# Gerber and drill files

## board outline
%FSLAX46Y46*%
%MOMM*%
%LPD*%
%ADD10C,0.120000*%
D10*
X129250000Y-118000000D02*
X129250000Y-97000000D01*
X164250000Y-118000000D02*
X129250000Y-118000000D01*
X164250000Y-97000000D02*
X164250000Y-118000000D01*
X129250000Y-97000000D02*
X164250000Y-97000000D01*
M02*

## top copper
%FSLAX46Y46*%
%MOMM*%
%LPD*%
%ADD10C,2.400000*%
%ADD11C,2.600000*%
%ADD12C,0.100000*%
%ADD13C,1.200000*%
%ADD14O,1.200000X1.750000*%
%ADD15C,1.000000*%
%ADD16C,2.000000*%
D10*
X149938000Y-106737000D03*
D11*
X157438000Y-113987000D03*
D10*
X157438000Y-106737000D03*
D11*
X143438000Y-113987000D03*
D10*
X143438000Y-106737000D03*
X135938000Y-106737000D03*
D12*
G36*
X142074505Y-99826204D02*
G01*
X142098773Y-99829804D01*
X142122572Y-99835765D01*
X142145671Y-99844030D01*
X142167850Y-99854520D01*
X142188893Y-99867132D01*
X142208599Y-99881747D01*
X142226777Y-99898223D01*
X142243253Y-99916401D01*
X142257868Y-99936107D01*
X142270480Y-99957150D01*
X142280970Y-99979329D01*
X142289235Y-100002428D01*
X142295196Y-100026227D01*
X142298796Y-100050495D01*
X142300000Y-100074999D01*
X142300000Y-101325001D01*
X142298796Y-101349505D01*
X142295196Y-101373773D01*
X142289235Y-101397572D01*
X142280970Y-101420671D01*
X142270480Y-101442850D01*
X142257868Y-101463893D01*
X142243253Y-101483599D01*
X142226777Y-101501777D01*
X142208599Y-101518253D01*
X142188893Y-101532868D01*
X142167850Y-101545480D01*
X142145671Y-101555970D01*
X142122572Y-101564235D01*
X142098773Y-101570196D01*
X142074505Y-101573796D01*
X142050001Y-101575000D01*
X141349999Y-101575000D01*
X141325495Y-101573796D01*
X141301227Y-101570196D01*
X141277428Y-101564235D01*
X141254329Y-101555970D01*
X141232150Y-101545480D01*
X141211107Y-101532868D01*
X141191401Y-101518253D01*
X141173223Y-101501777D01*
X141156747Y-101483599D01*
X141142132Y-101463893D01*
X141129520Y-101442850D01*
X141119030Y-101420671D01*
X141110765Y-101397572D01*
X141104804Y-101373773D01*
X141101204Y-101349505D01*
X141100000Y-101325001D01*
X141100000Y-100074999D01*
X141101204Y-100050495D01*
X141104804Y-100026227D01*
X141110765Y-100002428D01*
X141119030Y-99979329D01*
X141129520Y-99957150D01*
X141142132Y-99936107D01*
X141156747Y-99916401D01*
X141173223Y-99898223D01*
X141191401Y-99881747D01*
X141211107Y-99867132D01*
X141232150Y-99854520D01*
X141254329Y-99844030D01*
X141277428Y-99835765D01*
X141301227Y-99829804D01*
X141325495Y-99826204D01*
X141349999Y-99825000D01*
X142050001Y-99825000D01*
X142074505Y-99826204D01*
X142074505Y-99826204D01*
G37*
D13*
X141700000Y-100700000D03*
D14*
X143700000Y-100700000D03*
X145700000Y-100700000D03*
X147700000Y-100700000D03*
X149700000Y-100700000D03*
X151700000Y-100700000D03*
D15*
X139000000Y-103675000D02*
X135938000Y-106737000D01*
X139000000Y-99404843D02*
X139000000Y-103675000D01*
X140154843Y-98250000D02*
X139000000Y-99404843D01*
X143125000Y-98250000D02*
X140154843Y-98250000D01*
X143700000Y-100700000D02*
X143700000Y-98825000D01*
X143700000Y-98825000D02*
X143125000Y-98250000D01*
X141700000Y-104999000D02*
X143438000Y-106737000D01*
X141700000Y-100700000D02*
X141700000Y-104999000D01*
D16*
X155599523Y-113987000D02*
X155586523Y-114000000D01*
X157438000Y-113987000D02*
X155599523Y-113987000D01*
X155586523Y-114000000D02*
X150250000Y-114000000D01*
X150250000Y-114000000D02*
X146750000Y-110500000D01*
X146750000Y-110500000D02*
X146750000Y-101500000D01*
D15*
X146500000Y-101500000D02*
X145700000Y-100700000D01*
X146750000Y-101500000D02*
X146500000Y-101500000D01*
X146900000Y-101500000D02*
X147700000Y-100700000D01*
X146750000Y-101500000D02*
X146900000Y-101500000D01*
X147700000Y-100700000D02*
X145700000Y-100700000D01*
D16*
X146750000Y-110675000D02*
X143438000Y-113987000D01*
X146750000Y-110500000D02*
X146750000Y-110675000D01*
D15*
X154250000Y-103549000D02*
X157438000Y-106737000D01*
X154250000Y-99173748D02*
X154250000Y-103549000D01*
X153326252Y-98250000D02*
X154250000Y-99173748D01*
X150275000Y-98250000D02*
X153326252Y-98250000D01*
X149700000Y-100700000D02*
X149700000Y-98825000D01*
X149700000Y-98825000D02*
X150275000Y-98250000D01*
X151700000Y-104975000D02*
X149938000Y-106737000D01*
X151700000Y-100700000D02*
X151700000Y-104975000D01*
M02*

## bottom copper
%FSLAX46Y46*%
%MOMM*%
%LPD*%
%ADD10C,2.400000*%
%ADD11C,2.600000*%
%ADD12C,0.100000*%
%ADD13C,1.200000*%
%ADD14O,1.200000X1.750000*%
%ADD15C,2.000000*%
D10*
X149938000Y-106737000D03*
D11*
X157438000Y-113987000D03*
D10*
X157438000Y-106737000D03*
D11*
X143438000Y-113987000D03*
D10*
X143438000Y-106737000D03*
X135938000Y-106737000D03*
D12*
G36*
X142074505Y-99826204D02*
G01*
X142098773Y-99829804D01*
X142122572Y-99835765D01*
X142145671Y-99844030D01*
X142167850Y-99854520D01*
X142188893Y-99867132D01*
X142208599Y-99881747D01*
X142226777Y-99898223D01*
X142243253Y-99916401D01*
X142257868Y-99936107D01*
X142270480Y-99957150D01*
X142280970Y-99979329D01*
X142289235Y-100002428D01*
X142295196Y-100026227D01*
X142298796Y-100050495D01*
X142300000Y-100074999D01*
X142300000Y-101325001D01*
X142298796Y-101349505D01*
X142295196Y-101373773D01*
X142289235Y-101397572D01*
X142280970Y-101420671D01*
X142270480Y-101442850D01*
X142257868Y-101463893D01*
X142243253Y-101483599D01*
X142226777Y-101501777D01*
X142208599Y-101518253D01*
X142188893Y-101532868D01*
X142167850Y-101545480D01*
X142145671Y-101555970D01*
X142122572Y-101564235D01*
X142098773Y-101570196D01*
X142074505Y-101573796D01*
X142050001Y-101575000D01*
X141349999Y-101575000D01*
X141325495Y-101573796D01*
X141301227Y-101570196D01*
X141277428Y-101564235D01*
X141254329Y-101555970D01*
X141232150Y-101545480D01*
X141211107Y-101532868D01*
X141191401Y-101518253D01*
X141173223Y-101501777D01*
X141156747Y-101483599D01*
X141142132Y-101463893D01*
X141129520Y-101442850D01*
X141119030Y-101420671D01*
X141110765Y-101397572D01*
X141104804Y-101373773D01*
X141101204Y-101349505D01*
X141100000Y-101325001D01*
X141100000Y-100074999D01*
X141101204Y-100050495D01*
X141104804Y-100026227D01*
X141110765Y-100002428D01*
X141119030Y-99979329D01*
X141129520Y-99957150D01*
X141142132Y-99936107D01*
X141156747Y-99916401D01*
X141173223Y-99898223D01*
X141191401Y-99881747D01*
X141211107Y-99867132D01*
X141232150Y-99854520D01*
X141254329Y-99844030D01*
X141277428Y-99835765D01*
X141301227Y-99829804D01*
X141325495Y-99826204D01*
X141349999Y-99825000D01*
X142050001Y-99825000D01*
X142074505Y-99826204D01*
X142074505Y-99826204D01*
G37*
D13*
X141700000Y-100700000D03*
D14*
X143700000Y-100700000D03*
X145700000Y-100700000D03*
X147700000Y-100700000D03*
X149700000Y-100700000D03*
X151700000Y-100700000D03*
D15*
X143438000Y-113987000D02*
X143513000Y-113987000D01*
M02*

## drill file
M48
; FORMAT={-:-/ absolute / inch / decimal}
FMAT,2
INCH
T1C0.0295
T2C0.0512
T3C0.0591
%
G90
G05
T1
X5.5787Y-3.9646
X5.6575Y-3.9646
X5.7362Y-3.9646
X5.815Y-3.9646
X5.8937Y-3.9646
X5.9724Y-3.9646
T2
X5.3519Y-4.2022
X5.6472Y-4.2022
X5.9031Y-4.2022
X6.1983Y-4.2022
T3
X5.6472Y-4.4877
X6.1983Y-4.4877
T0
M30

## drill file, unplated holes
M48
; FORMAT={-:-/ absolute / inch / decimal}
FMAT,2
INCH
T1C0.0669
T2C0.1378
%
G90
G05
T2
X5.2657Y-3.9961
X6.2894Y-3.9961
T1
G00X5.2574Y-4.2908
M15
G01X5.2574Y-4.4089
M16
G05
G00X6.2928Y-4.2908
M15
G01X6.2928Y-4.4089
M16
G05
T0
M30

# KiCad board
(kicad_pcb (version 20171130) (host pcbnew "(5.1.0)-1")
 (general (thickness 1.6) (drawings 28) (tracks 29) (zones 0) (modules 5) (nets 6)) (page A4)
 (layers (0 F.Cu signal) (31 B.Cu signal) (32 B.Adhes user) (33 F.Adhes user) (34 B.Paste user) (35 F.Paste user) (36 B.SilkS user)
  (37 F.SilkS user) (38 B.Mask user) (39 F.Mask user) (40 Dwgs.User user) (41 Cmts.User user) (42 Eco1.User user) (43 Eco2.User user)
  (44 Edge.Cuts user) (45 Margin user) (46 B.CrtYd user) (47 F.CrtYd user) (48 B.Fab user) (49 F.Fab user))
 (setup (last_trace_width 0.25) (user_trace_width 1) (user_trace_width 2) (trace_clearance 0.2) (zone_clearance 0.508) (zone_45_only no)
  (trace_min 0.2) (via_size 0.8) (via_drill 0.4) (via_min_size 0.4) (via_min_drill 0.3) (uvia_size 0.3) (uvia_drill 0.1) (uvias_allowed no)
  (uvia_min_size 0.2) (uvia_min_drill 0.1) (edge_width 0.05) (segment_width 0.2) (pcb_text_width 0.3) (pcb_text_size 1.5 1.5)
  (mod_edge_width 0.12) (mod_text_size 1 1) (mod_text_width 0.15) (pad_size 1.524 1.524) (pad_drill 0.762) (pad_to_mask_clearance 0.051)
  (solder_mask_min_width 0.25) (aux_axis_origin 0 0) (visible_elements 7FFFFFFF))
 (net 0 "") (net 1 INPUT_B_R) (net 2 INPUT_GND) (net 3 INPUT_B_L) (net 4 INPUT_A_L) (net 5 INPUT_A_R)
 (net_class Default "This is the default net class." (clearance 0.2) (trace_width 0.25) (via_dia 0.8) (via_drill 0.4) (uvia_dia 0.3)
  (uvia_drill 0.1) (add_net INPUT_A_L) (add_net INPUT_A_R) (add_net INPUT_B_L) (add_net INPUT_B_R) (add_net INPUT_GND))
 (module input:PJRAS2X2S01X (layer F.Cu) (at 135.938 106.737)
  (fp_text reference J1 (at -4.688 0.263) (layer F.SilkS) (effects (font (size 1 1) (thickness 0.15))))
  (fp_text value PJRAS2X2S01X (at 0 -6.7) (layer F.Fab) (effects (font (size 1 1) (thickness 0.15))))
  (pad "" np_thru_hole oval (at 23.9 3.75) (size 1.7 4.7) (drill oval 1.7 4.7) (layers *.Cu *.Mask))
  (pad "" np_thru_hole oval (at -2.4 3.75) (size 1.7 4.7) (drill oval 1.7 4.7) (layers *.Cu *.Mask))
  (pad 4 thru_hole circle (at 14 0) (size 2.4 2.4) (drill 1.3) (layers *.Cu *.Mask) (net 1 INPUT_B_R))
  (pad 5 thru_hole circle (at 21.5 7.25) (size 2.6 2.6) (drill 1.5) (layers *.Cu *.Mask) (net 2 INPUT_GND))
  (pad 6 thru_hole circle (at 21.5 0) (size 2.4 2.4) (drill 1.3) (layers *.Cu *.Mask) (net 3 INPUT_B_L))
  (pad 2 thru_hole circle (at 7.5 7.25) (size 2.6 2.6) (drill 1.5) (layers *.Cu *.Mask) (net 2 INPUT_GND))
  (pad 3 thru_hole circle (at 7.5 0) (size 2.4 2.4) (drill 1.3) (layers *.Cu *.Mask) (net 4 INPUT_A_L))
  (pad 1 thru_hole circle (at 0 0) (size 2.4 2.4) (drill 1.3) (layers *.Cu *.Mask) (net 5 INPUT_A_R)))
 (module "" (layer F.Cu) (at 140.5 94.25)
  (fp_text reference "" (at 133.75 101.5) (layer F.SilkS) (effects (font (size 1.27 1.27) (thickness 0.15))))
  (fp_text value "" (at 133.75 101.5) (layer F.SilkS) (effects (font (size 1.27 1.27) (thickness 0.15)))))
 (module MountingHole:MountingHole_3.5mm (layer F.Cu) (at 133.75 101.5)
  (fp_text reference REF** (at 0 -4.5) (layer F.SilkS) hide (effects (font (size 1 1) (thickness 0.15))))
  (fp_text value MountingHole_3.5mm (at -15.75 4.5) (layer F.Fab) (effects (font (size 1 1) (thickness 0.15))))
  (pad 1 np_thru_hole circle (at 0 0) (size 3.5 3.5) (drill 3.5) (layers *.Cu *.Mask)))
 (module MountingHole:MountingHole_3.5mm (layer F.Cu) (at 159.75 101.5)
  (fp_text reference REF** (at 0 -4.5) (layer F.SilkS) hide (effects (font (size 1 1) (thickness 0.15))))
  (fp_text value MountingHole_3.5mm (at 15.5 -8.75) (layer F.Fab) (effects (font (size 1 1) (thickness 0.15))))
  (pad 1 np_thru_hole circle (at 0 0) (size 3.5 3.5) (drill 3.5) (layers *.Cu *.Mask)))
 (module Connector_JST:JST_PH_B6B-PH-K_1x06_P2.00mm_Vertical (layer F.Cu) (at 141.7 100.7)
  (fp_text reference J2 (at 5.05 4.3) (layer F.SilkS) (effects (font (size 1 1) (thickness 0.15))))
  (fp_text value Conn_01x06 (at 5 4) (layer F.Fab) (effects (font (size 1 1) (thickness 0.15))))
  (pad 1 thru_hole roundrect (at 0 0) (size 1.2 1.75) (drill 0.75) (layers *.Cu *.Mask) (roundrect_rratio 0.208333) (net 4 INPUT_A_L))
  (pad 2 thru_hole oval (at 2 0) (size 1.2 1.75) (drill 0.75) (layers *.Cu *.Mask) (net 5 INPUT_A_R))
  (pad 3 thru_hole oval (at 4 0) (size 1.2 1.75) (drill 0.75) (layers *.Cu *.Mask) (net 2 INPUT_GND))
  (pad 4 thru_hole oval (at 6 0) (size 1.2 1.75) (drill 0.75) (layers *.Cu *.Mask) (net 2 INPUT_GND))
  (pad 5 thru_hole oval (at 8 0) (size 1.2 1.75) (drill 0.75) (layers *.Cu *.Mask) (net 3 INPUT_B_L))
  (pad 6 thru_hole oval (at 10 0) (size 1.2 1.75) (drill 0.75) (layers *.Cu *.Mask) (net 1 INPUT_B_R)))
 (gr_line (start 129.25 118) (end 129.25 97) (layer Edge.Cuts) (width 0.12))
 (gr_line (start 164.25 118) (end 129.25 118) (layer Edge.Cuts) (width 0.12))
 (gr_line (start 164.25 97) (end 164.25 118) (layer Edge.Cuts) (width 0.12))
 (gr_line (start 129.25 97) (end 164.25 97) (layer Edge.Cuts) (width 0.12))
 (segment (start 139 103.675) (end 135.938 106.737) (width 1) (layer F.Cu) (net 5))
 (segment (start 139 99.404843) (end 139 103.675) (width 1) (layer F.Cu) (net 5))
 (segment (start 140.154843 98.25) (end 139 99.404843) (width 1) (layer F.Cu) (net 5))
 (segment (start 143.125 98.25) (end 140.154843 98.25) (width 1) (layer F.Cu) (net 5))
 (segment (start 143.7 100.7) (end 143.7 98.825) (width 1) (layer F.Cu) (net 5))
 (segment (start 143.7 98.825) (end 143.125 98.25) (width 1) (layer F.Cu) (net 5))
 (segment (start 141.7 104.999) (end 143.438 106.737) (width 1) (layer F.Cu) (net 4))
 (segment (start 141.7 100.7) (end 141.7 104.999) (width 1) (layer F.Cu) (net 4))
 (segment (start 155.599523 113.987) (end 155.586523 114) (width 2) (layer F.Cu) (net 2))
 (segment (start 157.438 113.987) (end 155.599523 113.987) (width 2) (layer F.Cu) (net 2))
 (segment (start 155.586523 114) (end 150.25 114) (width 2) (layer F.Cu) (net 2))
 (segment (start 150.25 114) (end 146.75 110.5) (width 2) (layer F.Cu) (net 2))
 (segment (start 146.75 110.5) (end 146.75 101.5) (width 2) (layer F.Cu) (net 2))
 (segment (start 146.5 101.5) (end 145.7 100.7) (width 1) (layer F.Cu) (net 2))
 (segment (start 146.75 101.5) (end 146.5 101.5) (width 1) (layer F.Cu) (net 2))
 (segment (start 146.9 101.5) (end 147.7 100.7) (width 1) (layer F.Cu) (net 2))
 (segment (start 146.75 101.5) (end 146.9 101.5) (width 1) (layer F.Cu) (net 2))
 (segment (start 143.438 113.987) (end 143.513 113.987) (width 2) (layer B.Cu) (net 2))
 (segment (start 147.7 100.7) (end 145.7 100.7) (width 1) (layer F.Cu) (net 2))
 (segment (start 146.75 110.675) (end 143.438 113.987) (width 2) (layer F.Cu) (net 2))
 (segment (start 146.75 110.5) (end 146.75 110.675) (width 2) (layer F.Cu) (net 2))
 (segment (start 154.25 103.549) (end 157.438 106.737) (width 1) (layer F.Cu) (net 3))
 (segment (start 154.25 99.173748) (end 154.25 103.549) (width 1) (layer F.Cu) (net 3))
 (segment (start 153.326252 98.25) (end 154.25 99.173748) (width 1) (layer F.Cu) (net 3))
 (segment (start 150.275 98.25) (end 153.326252 98.25) (width 1) (layer F.Cu) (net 3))
 (segment (start 149.7 100.7) (end 149.7 98.825) (width 1) (layer F.Cu) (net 3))
 (segment (start 149.7 98.825) (end 150.275 98.25) (width 1) (layer F.Cu) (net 3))
 (segment (start 151.7 104.975) (end 149.938 106.737) (width 1) (layer F.Cu) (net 1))
 (segment (start 151.7 100.7) (end 151.7 104.975) (width 1) (layer F.Cu) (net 1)))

